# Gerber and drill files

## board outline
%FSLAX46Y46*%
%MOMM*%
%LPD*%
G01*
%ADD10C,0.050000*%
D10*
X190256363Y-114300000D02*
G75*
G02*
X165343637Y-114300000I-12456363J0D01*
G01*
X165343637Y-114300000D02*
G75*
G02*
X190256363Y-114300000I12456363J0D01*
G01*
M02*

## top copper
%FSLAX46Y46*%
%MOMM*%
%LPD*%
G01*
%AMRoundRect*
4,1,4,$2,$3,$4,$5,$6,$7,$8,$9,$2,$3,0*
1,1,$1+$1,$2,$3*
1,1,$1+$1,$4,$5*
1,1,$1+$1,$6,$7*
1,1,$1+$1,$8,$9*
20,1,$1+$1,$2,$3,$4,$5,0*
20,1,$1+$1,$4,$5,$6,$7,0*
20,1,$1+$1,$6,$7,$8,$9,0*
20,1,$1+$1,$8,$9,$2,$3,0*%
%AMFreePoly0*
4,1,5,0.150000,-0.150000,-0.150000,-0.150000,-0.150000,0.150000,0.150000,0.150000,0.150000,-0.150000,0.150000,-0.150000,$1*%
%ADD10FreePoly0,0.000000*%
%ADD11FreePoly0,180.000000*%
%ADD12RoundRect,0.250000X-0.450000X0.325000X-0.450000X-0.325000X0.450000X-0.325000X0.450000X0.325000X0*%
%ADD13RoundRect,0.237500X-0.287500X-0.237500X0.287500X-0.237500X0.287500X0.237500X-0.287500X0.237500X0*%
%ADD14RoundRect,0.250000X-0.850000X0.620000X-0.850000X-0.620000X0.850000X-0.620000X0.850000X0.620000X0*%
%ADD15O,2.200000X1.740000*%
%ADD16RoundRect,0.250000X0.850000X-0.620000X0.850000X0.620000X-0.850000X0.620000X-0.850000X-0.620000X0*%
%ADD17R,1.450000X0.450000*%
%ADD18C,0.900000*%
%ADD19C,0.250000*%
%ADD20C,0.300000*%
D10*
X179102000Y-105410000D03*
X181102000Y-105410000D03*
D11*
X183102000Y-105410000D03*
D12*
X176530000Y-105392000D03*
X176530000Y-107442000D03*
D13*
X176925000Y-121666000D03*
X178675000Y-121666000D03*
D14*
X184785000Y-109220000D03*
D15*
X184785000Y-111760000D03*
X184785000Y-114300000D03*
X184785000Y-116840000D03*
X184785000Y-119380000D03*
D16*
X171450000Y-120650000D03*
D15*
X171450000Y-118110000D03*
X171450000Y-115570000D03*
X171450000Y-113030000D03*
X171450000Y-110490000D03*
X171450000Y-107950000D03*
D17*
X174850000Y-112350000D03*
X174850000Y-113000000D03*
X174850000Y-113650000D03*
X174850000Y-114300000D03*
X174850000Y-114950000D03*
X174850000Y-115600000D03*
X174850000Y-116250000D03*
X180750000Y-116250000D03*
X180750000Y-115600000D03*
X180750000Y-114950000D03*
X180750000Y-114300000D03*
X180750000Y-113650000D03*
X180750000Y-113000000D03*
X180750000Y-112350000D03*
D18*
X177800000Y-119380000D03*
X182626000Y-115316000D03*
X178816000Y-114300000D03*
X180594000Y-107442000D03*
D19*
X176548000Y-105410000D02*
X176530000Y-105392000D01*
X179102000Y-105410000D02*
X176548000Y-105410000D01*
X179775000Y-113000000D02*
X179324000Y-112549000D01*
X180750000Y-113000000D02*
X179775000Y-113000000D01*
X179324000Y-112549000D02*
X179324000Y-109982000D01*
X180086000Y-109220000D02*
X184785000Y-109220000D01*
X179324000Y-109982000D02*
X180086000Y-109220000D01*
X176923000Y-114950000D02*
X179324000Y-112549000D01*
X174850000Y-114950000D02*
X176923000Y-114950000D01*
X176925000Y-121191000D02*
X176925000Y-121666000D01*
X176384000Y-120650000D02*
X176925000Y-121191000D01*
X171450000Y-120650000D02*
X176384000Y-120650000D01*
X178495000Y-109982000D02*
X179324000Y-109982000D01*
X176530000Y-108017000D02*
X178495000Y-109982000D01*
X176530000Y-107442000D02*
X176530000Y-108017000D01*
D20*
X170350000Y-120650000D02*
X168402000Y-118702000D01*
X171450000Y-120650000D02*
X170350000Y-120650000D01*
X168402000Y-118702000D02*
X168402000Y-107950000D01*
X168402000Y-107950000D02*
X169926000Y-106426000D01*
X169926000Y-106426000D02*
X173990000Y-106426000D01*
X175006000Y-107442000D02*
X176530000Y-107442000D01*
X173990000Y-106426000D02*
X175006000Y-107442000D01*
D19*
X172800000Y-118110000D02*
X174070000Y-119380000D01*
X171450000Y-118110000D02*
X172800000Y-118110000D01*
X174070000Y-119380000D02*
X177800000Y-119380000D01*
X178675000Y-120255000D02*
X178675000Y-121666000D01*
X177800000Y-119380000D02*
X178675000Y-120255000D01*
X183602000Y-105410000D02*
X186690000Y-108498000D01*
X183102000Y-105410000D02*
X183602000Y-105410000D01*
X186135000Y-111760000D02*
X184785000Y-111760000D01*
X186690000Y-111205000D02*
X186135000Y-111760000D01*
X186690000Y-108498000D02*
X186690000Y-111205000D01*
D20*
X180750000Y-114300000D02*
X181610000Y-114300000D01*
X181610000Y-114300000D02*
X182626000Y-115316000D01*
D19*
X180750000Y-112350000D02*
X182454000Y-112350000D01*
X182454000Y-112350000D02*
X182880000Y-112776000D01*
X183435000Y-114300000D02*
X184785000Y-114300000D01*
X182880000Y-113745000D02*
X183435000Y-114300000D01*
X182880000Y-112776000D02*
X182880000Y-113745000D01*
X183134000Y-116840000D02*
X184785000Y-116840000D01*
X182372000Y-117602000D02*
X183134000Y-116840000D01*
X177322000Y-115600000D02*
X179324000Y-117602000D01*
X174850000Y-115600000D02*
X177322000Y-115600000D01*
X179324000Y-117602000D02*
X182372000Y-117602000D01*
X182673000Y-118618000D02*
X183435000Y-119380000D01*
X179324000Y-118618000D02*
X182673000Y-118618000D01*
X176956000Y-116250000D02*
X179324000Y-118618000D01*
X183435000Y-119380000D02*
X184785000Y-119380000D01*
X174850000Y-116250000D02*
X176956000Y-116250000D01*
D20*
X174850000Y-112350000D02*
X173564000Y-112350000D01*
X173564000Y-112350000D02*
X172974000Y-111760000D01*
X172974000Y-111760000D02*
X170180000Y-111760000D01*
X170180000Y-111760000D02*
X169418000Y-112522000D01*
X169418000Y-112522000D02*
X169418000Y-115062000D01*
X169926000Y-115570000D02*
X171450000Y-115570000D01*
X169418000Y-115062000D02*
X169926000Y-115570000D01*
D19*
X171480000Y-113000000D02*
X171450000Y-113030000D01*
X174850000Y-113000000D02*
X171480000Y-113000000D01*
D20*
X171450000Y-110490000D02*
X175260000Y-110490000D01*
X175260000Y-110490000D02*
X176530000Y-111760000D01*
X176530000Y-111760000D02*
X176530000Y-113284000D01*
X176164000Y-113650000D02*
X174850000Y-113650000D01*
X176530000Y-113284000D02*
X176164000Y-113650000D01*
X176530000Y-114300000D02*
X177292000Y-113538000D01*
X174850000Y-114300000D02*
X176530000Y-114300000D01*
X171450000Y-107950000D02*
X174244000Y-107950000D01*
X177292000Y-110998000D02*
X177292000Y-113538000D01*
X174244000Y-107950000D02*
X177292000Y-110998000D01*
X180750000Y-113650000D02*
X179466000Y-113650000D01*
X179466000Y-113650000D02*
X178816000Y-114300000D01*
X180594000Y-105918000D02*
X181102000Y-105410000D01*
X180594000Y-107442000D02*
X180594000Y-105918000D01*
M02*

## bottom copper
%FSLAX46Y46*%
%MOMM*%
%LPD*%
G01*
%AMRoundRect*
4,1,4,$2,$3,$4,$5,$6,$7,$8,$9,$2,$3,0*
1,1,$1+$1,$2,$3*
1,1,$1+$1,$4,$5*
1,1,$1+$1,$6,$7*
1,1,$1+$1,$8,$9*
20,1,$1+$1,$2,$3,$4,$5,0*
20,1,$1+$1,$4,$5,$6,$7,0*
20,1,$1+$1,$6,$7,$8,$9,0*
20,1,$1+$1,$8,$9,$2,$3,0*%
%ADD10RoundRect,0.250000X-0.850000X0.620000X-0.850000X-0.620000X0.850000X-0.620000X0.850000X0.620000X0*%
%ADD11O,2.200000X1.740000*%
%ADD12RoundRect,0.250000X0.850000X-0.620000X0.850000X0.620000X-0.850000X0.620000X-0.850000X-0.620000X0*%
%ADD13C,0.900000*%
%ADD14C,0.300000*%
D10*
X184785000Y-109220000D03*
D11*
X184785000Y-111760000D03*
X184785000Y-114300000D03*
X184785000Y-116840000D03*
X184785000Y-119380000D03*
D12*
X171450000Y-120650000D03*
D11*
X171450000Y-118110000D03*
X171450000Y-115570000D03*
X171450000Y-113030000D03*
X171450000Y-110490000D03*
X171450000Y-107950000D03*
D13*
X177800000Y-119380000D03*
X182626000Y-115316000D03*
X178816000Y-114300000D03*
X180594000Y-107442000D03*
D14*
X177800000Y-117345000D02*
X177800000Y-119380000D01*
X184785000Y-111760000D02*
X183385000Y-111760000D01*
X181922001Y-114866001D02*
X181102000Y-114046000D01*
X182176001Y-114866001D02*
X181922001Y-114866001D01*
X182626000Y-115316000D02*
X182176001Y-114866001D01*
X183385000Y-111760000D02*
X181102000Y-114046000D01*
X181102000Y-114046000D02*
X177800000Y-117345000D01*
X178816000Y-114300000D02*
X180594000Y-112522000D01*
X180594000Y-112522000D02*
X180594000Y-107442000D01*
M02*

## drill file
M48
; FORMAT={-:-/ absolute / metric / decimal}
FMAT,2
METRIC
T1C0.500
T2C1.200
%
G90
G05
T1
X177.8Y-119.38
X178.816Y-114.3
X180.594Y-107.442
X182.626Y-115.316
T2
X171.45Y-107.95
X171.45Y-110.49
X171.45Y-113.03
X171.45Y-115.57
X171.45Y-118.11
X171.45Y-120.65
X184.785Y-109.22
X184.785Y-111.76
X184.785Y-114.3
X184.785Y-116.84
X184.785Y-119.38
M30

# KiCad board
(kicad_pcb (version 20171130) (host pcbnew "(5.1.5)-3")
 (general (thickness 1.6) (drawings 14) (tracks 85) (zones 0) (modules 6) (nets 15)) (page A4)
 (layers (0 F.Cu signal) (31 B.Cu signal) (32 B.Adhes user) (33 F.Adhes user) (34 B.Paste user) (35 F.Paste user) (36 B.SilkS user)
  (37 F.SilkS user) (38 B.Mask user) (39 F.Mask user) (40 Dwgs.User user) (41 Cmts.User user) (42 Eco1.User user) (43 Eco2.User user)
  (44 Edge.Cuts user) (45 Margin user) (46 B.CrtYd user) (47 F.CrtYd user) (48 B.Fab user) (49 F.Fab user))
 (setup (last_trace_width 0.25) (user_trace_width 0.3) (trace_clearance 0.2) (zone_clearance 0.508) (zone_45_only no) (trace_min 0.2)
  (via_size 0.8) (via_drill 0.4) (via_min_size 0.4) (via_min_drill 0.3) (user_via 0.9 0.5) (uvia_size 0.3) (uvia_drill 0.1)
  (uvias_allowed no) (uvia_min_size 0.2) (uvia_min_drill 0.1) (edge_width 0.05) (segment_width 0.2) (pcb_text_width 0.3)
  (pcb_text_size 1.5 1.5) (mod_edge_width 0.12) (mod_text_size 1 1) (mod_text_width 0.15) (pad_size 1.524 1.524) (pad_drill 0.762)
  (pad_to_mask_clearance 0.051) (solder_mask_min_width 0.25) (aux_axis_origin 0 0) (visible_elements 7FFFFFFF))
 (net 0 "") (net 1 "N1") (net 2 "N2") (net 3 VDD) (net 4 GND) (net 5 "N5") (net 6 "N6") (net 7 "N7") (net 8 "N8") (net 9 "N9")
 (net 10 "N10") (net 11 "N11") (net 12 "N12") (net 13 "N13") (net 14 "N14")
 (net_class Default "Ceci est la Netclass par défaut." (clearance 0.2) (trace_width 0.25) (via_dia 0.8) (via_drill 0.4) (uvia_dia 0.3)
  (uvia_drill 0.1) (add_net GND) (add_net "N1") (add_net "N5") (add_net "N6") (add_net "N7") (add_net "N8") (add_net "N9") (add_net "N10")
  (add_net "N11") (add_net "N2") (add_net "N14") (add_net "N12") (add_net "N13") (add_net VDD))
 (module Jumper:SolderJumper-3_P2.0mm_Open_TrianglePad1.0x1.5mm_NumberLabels (layer F.Cu) (at 181.102 105.41)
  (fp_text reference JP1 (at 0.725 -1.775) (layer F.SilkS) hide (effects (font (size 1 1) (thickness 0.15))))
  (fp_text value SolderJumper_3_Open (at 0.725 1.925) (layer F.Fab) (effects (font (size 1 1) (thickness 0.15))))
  (pad "" smd rect (at 1.2 0) (size 1.5 1.5) (layers F.Mask)) (pad "" smd rect (at -1.2 0) (size 1.5 1.5) (layers F.Mask))
  (pad 1 smd custom (at -2 0) (size 0.3 0.3) (layers F.Cu F.Mask) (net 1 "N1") (zone_connect 2) (options (clearance outline) (anchor rect))
   (primitives))
  (pad 2 smd custom (at 0 0) (size 0.3 0.3) (layers F.Cu) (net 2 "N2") (zone_connect 2) (options (clearance outline) (anchor rect))
   (primitives))
  (pad 3 smd custom (at 2 0 180) (size 0.3 0.3) (layers F.Cu F.Mask) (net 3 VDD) (zone_connect 2)
   (options (clearance outline) (anchor rect)) (primitives)))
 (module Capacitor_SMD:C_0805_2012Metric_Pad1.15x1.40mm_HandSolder (layer F.Cu) (at 176.53 106.417 270)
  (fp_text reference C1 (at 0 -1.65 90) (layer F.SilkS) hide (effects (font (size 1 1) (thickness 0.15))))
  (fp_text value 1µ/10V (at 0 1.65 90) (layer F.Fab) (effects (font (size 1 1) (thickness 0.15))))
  (pad 1 smd roundrect (at -1.025 0 270) (size 1.15 1.4) (layers F.Cu F.Paste F.Mask) (roundrect_rratio 0.217391) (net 1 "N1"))
  (pad 2 smd roundrect (at 1.025 0 270) (size 1.15 1.4) (layers F.Cu F.Paste F.Mask) (roundrect_rratio 0.217391) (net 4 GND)))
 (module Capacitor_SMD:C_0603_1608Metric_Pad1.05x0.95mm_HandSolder (layer F.Cu) (at 177.8 121.666)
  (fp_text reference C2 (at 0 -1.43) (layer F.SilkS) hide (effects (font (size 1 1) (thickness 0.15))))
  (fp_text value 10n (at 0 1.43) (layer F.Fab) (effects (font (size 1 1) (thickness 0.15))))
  (pad 1 smd roundrect (at -0.875 0) (size 1.05 0.95) (layers F.Cu F.Paste F.Mask) (roundrect_rratio 0.25) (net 4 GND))
  (pad 2 smd roundrect (at 0.875 0) (size 1.05 0.95) (layers F.Cu F.Paste F.Mask) (roundrect_rratio 0.25) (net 3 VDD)))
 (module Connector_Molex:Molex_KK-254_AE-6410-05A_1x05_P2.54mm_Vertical (layer B.Cu) (at 184.785 109.22 270)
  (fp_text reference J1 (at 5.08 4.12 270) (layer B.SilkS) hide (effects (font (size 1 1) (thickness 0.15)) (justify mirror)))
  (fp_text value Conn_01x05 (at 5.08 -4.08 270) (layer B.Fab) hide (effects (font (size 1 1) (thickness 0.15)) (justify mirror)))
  (pad 1 thru_hole roundrect (at 0 0 270) (size 1.74 2.2) (drill 1.2) (layers *.Cu *.Mask) (roundrect_rratio 0.143678) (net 4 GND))
  (pad 2 thru_hole oval (at 2.54 0 270) (size 1.74 2.2) (drill 1.2) (layers *.Cu *.Mask) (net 3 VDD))
  (pad 3 thru_hole oval (at 5.08 0 270) (size 1.74 2.2) (drill 1.2) (layers *.Cu *.Mask) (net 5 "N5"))
  (pad 4 thru_hole oval (at 7.62 0 270) (size 1.74 2.2) (drill 1.2) (layers *.Cu *.Mask) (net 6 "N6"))
  (pad 5 thru_hole oval (at 10.16 0 270) (size 1.74 2.2) (drill 1.2) (layers *.Cu *.Mask) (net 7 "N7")))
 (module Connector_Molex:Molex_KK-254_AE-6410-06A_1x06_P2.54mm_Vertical (layer B.Cu) (at 171.45 120.65 90)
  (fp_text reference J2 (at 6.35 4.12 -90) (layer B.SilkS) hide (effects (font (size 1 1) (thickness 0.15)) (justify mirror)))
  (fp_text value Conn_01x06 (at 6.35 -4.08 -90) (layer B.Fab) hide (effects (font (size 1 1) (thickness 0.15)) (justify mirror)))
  (pad 1 thru_hole roundrect (at 0 0 90) (size 1.74 2.2) (drill 1.2) (layers *.Cu *.Mask) (roundrect_rratio 0.143678) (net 4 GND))
  (pad 2 thru_hole oval (at 2.54 0 90) (size 1.74 2.2) (drill 1.2) (layers *.Cu *.Mask) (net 3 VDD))
  (pad 3 thru_hole oval (at 5.08 0 90) (size 1.74 2.2) (drill 1.2) (layers *.Cu *.Mask) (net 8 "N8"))
  (pad 4 thru_hole oval (at 7.62 0 90) (size 1.74 2.2) (drill 1.2) (layers *.Cu *.Mask) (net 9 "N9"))
  (pad 5 thru_hole oval (at 10.16 0 90) (size 1.74 2.2) (drill 1.2) (layers *.Cu *.Mask) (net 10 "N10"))
  (pad 6 thru_hole oval (at 12.7 0 90) (size 1.74 2.2) (drill 1.2) (layers *.Cu *.Mask) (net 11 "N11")))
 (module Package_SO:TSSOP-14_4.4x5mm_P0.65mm (layer F.Cu) (at 177.8 114.3)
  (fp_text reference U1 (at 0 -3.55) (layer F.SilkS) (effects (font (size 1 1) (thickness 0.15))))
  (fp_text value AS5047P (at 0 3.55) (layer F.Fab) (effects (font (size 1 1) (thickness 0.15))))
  (pad 1 smd rect (at -2.95 -1.95) (size 1.45 0.45) (layers F.Cu F.Paste F.Mask) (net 8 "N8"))
  (pad 2 smd rect (at -2.95 -1.3) (size 1.45 0.45) (layers F.Cu F.Paste F.Mask) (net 9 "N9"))
  (pad 3 smd rect (at -2.95 -0.65) (size 1.45 0.45) (layers F.Cu F.Paste F.Mask) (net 10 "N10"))
  (pad 4 smd rect (at -2.95 0) (size 1.45 0.45) (layers F.Cu F.Paste F.Mask) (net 11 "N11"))
  (pad 5 smd rect (at -2.95 0.65) (size 1.45 0.45) (layers F.Cu F.Paste F.Mask) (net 4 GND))
  (pad 6 smd rect (at -2.95 1.3) (size 1.45 0.45) (layers F.Cu F.Paste F.Mask) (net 6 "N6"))
  (pad 7 smd rect (at -2.95 1.95) (size 1.45 0.45) (layers F.Cu F.Paste F.Mask) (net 7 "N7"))
  (pad 8 smd rect (at 2.95 1.95) (size 1.45 0.45) (layers F.Cu F.Paste F.Mask) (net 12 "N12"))
  (pad 9 smd rect (at 2.95 1.3) (size 1.45 0.45) (layers F.Cu F.Paste F.Mask) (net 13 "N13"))
  (pad 10 smd rect (at 2.95 0.65) (size 1.45 0.45) (layers F.Cu F.Paste F.Mask) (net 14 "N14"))
  (pad 11 smd rect (at 2.95 0) (size 1.45 0.45) (layers F.Cu F.Paste F.Mask) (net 3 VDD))
  (pad 12 smd rect (at 2.95 -0.65) (size 1.45 0.45) (layers F.Cu F.Paste F.Mask) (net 2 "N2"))
  (pad 13 smd rect (at 2.95 -1.3) (size 1.45 0.45) (layers F.Cu F.Paste F.Mask) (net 4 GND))
  (pad 14 smd rect (at 2.95 -1.95) (size 1.45 0.45) (layers F.Cu F.Paste F.Mask) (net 5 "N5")))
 (gr_circle (center 177.8 114.3) (end 189.738 117.856) (layer Edge.Cuts) (width 0.05))
 (segment (start 176.548 105.41) (end 176.53 105.392) (width 0.25) (layer F.Cu) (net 1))
 (segment (start 179.102 105.41) (end 176.548 105.41) (width 0.25) (layer F.Cu) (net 1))
 (segment (start 179.775 113) (end 179.324 112.549) (width 0.25) (layer F.Cu) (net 4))
 (segment (start 180.75 113) (end 179.775 113) (width 0.25) (layer F.Cu) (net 4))
 (segment (start 179.324 112.549) (end 179.324 109.982) (width 0.25) (layer F.Cu) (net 4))
 (segment (start 180.086 109.22) (end 184.785 109.22) (width 0.25) (layer F.Cu) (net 4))
 (segment (start 179.324 109.982) (end 180.086 109.22) (width 0.25) (layer F.Cu) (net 4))
 (segment (start 176.923 114.95) (end 179.324 112.549) (width 0.25) (layer F.Cu) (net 4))
 (segment (start 174.85 114.95) (end 176.923 114.95) (width 0.25) (layer F.Cu) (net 4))
 (segment (start 176.925 121.191) (end 176.925 121.666) (width 0.25) (layer F.Cu) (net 4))
 (segment (start 176.384 120.65) (end 176.925 121.191) (width 0.25) (layer F.Cu) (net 4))
 (segment (start 171.45 120.65) (end 176.384 120.65) (width 0.25) (layer F.Cu) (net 4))
 (segment (start 178.495 109.982) (end 179.324 109.982) (width 0.25) (layer F.Cu) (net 4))
 (segment (start 176.53 108.017) (end 178.495 109.982) (width 0.25) (layer F.Cu) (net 4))
 (segment (start 176.53 107.442) (end 176.53 108.017) (width 0.25) (layer F.Cu) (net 4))
 (segment (start 170.35 120.65) (end 168.402 118.702) (width 0.3) (layer F.Cu) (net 4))
 (segment (start 171.45 120.65) (end 170.35 120.65) (width 0.3) (layer F.Cu) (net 4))
 (segment (start 168.402 118.702) (end 168.402 107.95) (width 0.3) (layer F.Cu) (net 4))
 (segment (start 168.402 107.95) (end 169.926 106.426) (width 0.3) (layer F.Cu) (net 4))
 (segment (start 169.926 106.426) (end 173.99 106.426) (width 0.3) (layer F.Cu) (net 4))
 (segment (start 175.006 107.442) (end 176.53 107.442) (width 0.3) (layer F.Cu) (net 4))
 (segment (start 173.99 106.426) (end 175.006 107.442) (width 0.3) (layer F.Cu) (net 4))
 (segment (start 172.8 118.11) (end 174.07 119.38) (width 0.25) (layer F.Cu) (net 3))
 (segment (start 171.45 118.11) (end 172.8 118.11) (width 0.25) (layer F.Cu) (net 3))
 (segment (start 174.07 119.38) (end 177.8 119.38) (width 0.25) (layer F.Cu) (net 3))
 (segment (start 178.675 120.255) (end 178.675 121.666) (width 0.25) (layer F.Cu) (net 3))
 (segment (start 177.8 119.38) (end 178.675 120.255) (width 0.25) (layer F.Cu) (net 3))
 (segment (start 183.602 105.41) (end 186.69 108.498) (width 0.25) (layer F.Cu) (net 3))
 (segment (start 183.102 105.41) (end 183.602 105.41) (width 0.25) (layer F.Cu) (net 3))
 (segment (start 186.135 111.76) (end 184.785 111.76) (width 0.25) (layer F.Cu) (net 3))
 (segment (start 186.69 111.205) (end 186.135 111.76) (width 0.25) (layer F.Cu) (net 3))
 (segment (start 186.69 108.498) (end 186.69 111.205) (width 0.25) (layer F.Cu) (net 3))
 (via (at 177.8 119.38) (size 0.9) (drill 0.5) (layers F.Cu B.Cu) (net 3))
 (segment (start 177.8 117.345) (end 177.8 119.38) (width 0.3) (layer B.Cu) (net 3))
 (segment (start 184.785 111.76) (end 183.385 111.76) (width 0.3) (layer B.Cu) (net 3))
 (via (at 182.626 115.316) (size 0.9) (drill 0.5) (layers F.Cu B.Cu) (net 3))
 (segment (start 180.75 114.3) (end 181.61 114.3) (width 0.3) (layer F.Cu) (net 3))
 (segment (start 181.61 114.3) (end 182.626 115.316) (width 0.3) (layer F.Cu) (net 3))
 (segment (start 181.922001 114.866001) (end 181.102 114.046) (width 0.3) (layer B.Cu) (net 3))
 (segment (start 182.176001 114.866001) (end 181.922001 114.866001) (width 0.3) (layer B.Cu) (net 3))
 (segment (start 182.626 115.316) (end 182.176001 114.866001) (width 0.3) (layer B.Cu) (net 3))
 (segment (start 183.385 111.76) (end 181.102 114.046) (width 0.3) (layer B.Cu) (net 3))
 (segment (start 181.102 114.046) (end 177.8 117.345) (width 0.3) (layer B.Cu) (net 3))
 (segment (start 180.75 112.35) (end 182.454 112.35) (width 0.25) (layer F.Cu) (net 5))
 (segment (start 182.454 112.35) (end 182.88 112.776) (width 0.25) (layer F.Cu) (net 5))
 (segment (start 183.435 114.3) (end 184.785 114.3) (width 0.25) (layer F.Cu) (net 5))
 (segment (start 182.88 113.745) (end 183.435 114.3) (width 0.25) (layer F.Cu) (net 5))
 (segment (start 182.88 112.776) (end 182.88 113.745) (width 0.25) (layer F.Cu) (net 5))
 (segment (start 183.134 116.84) (end 184.785 116.84) (width 0.25) (layer F.Cu) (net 6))
 (segment (start 182.372 117.602) (end 183.134 116.84) (width 0.25) (layer F.Cu) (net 6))
 (segment (start 177.322 115.6) (end 179.324 117.602) (width 0.25) (layer F.Cu) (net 6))
 (segment (start 174.85 115.6) (end 177.322 115.6) (width 0.25) (layer F.Cu) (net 6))
 (segment (start 179.324 117.602) (end 182.372 117.602) (width 0.25) (layer F.Cu) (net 6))
 (segment (start 182.673 118.618) (end 183.435 119.38) (width 0.25) (layer F.Cu) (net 7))
 (segment (start 179.324 118.618) (end 182.673 118.618) (width 0.25) (layer F.Cu) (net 7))
 (segment (start 176.956 116.25) (end 179.324 118.618) (width 0.25) (layer F.Cu) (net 7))
 (segment (start 183.435 119.38) (end 184.785 119.38) (width 0.25) (layer F.Cu) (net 7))
 (segment (start 174.85 116.25) (end 176.956 116.25) (width 0.25) (layer F.Cu) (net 7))
 (segment (start 174.85 112.35) (end 173.564 112.35) (width 0.3) (layer F.Cu) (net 8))
 (segment (start 173.564 112.35) (end 172.974 111.76) (width 0.3) (layer F.Cu) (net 8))
 (segment (start 172.974 111.76) (end 170.18 111.76) (width 0.3) (layer F.Cu) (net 8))
 (segment (start 170.18 111.76) (end 169.418 112.522) (width 0.3) (layer F.Cu) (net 8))
 (segment (start 169.418 112.522) (end 169.418 115.062) (width 0.3) (layer F.Cu) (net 8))
 (segment (start 169.926 115.57) (end 171.45 115.57) (width 0.3) (layer F.Cu) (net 8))
 (segment (start 169.418 115.062) (end 169.926 115.57) (width 0.3) (layer F.Cu) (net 8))
 (segment (start 171.48 113) (end 171.45 113.03) (width 0.25) (layer F.Cu) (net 9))
 (segment (start 174.85 113) (end 171.48 113) (width 0.25) (layer F.Cu) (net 9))
 (segment (start 171.45 110.49) (end 175.26 110.49) (width 0.3) (layer F.Cu) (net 10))
 (segment (start 175.26 110.49) (end 176.53 111.76) (width 0.3) (layer F.Cu) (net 10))
 (segment (start 176.53 111.76) (end 176.53 113.284) (width 0.3) (layer F.Cu) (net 10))
 (segment (start 176.164 113.65) (end 174.85 113.65) (width 0.3) (layer F.Cu) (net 10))
 (segment (start 176.53 113.284) (end 176.164 113.65) (width 0.3) (layer F.Cu) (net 10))
 (segment (start 176.53 114.3) (end 177.292 113.538) (width 0.3) (layer F.Cu) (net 11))
 (segment (start 174.85 114.3) (end 176.53 114.3) (width 0.3) (layer F.Cu) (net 11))
 (segment (start 171.45 107.95) (end 174.244 107.95) (width 0.3) (layer F.Cu) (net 11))
 (segment (start 177.292 110.998) (end 177.292 113.538) (width 0.3) (layer F.Cu) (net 11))
 (segment (start 174.244 107.95) (end 177.292 110.998) (width 0.3) (layer F.Cu) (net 11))
 (segment (start 180.75 113.65) (end 179.466 113.65) (width 0.3) (layer F.Cu) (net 2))
 (via (at 178.816 114.3) (size 0.9) (drill 0.5) (layers F.Cu B.Cu) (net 2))
 (segment (start 179.466 113.65) (end 178.816 114.3) (width 0.3) (layer F.Cu) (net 2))
 (via (at 180.594 107.442) (size 0.9) (drill 0.5) (layers F.Cu B.Cu) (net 2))
 (segment (start 178.816 114.3) (end 180.594 112.522) (width 0.3) (layer B.Cu) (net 2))
 (segment (start 180.594 112.522) (end 180.594 107.442) (width 0.3) (layer B.Cu) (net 2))
 (segment (start 180.594 105.918) (end 181.102 105.41) (width 0.3) (layer F.Cu) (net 2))
 (segment (start 180.594 107.442) (end 180.594 105.918) (width 0.3) (layer F.Cu) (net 2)))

